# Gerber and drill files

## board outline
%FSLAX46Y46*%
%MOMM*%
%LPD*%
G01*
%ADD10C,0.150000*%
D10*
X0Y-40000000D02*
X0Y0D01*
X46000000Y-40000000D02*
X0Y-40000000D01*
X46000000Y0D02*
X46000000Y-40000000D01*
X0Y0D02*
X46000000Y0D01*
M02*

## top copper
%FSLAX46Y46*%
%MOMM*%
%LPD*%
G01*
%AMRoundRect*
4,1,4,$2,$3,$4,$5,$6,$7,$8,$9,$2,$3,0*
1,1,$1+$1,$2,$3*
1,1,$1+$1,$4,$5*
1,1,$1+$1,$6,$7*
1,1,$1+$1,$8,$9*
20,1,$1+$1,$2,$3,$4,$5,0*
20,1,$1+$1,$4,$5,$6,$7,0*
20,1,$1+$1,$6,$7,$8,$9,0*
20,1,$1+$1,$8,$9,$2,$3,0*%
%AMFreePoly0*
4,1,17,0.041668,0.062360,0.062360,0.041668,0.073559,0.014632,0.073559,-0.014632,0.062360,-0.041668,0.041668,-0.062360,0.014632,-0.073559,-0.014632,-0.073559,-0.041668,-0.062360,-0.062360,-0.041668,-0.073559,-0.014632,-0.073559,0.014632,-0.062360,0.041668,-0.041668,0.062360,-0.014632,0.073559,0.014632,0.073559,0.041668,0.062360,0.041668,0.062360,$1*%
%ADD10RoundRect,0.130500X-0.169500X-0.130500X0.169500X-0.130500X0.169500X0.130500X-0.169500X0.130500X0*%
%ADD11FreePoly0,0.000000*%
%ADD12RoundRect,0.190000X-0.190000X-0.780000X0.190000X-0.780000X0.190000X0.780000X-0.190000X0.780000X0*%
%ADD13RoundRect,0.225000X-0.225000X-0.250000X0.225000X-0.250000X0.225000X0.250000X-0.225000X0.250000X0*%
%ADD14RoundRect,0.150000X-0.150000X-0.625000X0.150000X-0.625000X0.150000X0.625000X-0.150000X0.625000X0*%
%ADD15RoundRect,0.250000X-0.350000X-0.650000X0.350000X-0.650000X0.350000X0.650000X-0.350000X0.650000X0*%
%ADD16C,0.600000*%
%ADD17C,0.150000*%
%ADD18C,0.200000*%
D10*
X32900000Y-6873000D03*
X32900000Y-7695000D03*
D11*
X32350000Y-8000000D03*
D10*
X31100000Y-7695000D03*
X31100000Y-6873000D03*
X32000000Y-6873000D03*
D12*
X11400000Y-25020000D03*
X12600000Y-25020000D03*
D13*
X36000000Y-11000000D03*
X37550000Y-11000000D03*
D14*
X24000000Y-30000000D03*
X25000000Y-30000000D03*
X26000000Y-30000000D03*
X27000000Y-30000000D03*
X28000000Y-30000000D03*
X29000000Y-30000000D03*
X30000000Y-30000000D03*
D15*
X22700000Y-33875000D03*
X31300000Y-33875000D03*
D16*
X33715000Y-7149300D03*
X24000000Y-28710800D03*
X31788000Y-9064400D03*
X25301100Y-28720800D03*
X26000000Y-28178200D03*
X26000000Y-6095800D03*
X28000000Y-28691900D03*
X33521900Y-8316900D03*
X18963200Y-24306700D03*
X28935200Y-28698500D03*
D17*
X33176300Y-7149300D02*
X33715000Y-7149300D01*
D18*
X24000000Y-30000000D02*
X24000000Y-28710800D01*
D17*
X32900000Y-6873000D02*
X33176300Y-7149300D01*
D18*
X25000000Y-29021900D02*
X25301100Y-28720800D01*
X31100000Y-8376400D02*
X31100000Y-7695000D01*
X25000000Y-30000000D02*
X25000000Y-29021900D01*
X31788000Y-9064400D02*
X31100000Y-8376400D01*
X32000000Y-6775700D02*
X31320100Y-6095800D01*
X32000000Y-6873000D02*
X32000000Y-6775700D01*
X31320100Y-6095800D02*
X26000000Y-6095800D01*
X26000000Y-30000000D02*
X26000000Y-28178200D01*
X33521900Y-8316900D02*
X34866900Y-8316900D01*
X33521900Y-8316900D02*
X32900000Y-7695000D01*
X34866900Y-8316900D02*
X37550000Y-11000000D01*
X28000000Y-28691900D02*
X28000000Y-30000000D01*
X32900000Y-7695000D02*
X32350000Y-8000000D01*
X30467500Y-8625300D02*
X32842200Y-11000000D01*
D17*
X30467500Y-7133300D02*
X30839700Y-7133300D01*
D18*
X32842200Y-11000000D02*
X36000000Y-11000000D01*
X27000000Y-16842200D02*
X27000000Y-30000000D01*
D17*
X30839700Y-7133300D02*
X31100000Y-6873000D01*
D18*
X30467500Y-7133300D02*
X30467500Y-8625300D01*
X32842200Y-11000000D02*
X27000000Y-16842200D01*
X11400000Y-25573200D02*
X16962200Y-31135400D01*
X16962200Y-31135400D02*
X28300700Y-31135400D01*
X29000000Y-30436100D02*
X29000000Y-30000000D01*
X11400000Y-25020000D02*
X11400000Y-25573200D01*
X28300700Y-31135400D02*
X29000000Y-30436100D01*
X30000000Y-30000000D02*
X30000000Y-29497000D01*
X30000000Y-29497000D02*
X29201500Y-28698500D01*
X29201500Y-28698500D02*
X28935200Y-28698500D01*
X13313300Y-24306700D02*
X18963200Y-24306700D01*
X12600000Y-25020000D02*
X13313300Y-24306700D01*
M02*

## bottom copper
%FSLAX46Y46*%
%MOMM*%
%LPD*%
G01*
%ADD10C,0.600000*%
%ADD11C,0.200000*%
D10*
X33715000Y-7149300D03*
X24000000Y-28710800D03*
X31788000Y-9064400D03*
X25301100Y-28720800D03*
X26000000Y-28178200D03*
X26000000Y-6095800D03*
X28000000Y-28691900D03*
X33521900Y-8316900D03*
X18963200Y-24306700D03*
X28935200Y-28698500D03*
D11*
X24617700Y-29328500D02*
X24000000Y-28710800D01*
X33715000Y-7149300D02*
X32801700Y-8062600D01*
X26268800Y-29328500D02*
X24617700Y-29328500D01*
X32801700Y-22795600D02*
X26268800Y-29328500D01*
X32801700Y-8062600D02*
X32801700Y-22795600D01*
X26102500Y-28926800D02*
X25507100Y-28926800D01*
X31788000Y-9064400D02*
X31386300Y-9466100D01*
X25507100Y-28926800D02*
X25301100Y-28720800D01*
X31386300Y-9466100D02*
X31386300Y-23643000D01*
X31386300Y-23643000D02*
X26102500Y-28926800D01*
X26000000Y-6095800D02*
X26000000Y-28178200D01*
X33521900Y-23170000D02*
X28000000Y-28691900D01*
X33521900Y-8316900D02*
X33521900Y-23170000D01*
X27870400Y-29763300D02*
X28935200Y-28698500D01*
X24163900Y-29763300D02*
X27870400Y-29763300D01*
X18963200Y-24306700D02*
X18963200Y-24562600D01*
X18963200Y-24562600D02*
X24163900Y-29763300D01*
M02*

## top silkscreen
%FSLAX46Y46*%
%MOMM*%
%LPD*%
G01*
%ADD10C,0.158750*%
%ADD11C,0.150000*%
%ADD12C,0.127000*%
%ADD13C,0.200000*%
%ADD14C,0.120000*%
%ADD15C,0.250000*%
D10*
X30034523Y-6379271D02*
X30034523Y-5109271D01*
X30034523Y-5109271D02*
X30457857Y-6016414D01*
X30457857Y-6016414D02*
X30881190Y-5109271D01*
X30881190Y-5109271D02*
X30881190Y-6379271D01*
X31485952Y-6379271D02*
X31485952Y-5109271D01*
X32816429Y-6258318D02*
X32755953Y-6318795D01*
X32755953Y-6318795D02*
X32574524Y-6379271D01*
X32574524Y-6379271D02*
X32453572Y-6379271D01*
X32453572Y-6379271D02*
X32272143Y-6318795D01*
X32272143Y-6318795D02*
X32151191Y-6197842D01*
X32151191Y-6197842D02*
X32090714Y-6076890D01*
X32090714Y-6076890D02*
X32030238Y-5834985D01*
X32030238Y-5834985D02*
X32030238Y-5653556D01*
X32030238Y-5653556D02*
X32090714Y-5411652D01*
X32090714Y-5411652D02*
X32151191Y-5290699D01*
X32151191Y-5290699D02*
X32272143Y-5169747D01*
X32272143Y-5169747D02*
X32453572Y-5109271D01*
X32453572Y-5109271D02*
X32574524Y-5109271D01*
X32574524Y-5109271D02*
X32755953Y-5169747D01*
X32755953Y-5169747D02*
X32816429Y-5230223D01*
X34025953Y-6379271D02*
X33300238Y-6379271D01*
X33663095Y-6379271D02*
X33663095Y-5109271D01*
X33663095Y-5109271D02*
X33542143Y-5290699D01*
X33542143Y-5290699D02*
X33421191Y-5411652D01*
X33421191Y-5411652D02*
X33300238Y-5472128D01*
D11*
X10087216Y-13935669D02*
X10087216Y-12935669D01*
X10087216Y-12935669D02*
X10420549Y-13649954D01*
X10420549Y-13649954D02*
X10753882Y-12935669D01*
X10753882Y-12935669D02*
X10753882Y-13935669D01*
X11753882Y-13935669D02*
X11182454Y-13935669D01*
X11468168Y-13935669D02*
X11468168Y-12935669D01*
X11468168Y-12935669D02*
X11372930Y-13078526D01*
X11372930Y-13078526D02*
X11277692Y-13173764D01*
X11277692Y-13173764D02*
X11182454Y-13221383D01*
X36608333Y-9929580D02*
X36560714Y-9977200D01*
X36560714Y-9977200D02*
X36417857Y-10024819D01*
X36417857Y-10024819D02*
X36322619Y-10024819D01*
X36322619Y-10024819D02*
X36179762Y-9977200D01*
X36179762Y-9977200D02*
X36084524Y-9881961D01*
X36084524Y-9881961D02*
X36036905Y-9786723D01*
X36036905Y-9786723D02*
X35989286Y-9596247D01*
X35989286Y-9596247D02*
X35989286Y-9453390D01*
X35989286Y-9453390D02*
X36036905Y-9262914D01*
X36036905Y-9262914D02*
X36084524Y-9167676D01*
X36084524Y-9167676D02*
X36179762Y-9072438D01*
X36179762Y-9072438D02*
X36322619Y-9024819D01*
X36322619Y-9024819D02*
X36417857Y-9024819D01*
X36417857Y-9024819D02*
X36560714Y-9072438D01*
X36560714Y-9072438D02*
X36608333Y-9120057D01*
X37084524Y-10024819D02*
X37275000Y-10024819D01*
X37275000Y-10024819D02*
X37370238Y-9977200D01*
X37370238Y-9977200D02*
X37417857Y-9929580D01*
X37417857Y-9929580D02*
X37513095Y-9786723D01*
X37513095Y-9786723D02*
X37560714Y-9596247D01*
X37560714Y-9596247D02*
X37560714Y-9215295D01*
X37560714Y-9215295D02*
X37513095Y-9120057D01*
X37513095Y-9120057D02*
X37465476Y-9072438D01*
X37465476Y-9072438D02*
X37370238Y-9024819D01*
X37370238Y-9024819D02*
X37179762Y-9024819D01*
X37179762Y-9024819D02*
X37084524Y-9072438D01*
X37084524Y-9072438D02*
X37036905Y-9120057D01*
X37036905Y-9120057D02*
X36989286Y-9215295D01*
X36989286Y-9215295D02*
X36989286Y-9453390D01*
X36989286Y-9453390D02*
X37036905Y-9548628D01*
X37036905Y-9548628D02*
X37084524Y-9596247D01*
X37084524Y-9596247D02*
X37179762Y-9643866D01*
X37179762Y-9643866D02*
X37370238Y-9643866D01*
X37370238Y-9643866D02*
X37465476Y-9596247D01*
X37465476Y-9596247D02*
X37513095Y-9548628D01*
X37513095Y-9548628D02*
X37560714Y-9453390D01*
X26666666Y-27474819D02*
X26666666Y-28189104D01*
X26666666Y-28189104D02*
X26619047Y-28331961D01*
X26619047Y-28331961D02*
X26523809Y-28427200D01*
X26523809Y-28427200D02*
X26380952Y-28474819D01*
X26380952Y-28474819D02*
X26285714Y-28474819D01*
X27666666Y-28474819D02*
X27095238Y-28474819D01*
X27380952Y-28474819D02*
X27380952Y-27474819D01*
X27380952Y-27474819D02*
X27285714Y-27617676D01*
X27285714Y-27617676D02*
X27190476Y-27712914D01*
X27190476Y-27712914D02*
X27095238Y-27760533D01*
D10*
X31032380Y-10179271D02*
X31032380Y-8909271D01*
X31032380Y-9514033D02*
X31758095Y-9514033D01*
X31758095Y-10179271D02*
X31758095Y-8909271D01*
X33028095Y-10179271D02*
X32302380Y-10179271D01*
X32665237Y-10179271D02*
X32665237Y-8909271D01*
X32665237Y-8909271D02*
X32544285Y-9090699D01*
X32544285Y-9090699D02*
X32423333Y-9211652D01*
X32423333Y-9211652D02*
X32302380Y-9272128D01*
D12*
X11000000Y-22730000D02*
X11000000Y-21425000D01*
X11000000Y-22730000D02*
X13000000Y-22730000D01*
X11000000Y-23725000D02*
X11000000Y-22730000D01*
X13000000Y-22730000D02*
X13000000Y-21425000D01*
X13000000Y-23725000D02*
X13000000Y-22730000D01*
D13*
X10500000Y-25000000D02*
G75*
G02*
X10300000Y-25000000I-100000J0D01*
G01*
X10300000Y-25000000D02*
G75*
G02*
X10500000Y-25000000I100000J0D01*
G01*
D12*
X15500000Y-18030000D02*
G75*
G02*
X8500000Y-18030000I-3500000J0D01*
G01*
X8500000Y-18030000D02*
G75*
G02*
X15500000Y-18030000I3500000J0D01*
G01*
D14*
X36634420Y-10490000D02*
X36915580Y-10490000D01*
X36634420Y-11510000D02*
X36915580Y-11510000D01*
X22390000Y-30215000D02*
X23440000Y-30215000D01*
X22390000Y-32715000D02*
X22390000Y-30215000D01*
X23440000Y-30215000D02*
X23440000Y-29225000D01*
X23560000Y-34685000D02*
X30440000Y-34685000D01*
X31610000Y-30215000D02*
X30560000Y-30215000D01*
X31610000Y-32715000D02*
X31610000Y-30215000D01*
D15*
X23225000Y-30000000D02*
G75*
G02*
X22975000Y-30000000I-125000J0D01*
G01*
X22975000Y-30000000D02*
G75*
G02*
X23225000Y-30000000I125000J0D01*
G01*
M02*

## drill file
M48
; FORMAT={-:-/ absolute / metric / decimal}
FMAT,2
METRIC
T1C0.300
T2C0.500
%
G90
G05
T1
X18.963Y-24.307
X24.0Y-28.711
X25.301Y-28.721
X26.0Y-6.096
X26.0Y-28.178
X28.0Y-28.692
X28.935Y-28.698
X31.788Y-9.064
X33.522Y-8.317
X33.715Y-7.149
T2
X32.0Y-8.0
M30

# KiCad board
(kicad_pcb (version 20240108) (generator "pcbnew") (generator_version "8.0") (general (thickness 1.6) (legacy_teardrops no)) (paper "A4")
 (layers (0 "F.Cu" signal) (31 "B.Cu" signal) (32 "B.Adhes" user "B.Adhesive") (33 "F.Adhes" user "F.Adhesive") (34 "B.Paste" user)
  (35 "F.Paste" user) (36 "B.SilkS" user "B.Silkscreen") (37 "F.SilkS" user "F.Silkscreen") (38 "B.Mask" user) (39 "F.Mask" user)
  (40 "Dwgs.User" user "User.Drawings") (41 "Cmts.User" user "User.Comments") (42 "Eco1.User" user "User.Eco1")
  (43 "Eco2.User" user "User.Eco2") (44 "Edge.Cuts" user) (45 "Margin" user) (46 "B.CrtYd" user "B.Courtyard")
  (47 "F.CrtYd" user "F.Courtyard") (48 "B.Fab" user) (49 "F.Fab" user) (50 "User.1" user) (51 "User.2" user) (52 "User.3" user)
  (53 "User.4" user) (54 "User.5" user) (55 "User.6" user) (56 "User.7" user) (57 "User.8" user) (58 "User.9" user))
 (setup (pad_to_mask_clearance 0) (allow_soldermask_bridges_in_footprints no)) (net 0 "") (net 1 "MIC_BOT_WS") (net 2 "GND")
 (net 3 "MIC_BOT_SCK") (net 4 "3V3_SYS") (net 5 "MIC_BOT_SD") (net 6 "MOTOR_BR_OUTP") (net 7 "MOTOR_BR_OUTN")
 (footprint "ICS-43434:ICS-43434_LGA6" (layer "F.Cu") (at 32 8)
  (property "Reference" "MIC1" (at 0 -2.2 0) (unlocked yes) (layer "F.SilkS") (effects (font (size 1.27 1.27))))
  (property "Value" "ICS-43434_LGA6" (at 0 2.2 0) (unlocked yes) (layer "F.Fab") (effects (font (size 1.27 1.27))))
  (pad "1" smd roundrect (at 0.9 -1.127) (size 0.6 0.522) (layers "F.Cu" "F.Paste" "F.Mask") (roundrect_rratio 0.25) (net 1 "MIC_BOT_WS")
   (thermal_bridge_angle 45))
  (pad "2" smd roundrect (at 0.9 -0.305) (size 0.6 0.522) (layers "F.Cu" "F.Paste" "F.Mask") (roundrect_rratio 0.25) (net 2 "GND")
   (thermal_bridge_angle 45))
  (pad "3" smd custom (at 0.35 0) (size 0.15 0.15) (layers "F.Cu" "F.Mask") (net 2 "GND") (options (clearance outline) (anchor circle))
   (primitives))
  (pad "4" smd roundrect (at -0.9 -0.305) (size 0.6 0.522) (layers "F.Cu" "F.Paste" "F.Mask") (roundrect_rratio 0.25) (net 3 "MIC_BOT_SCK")
   (thermal_bridge_angle 45))
  (pad "5" smd roundrect (at -0.9 -1.127) (size 0.6 0.522) (layers "F.Cu" "F.Paste" "F.Mask") (roundrect_rratio 0.25) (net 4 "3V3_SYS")
   (thermal_bridge_angle 45))
  (pad "6" smd roundrect (at 0 -1.127) (size 0.6 0.522) (layers "F.Cu" "F.Paste" "F.Mask") (roundrect_rratio 0.25) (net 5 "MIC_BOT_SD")
   (thermal_bridge_angle 45)))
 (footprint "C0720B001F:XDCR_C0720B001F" (layer "F.Cu") (at 12 20)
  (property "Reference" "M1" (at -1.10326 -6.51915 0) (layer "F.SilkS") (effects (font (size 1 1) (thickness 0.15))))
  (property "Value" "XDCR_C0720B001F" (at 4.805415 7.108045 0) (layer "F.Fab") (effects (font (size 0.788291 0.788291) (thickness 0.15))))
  (fp_line (start -1 2.73) (end -1 1.425) (stroke (width 0.127) (type solid)) (layer "F.SilkS"))
  (fp_line (start -1 2.73) (end 1 2.73) (stroke (width 0.127) (type solid)) (layer "F.SilkS"))
  (fp_line (start -1 3.725) (end -1 2.73) (stroke (width 0.127) (type solid)) (layer "F.SilkS"))
  (fp_line (start 1 2.73) (end 1 1.425) (stroke (width 0.127) (type solid)) (layer "F.SilkS"))
  (fp_line (start 1 3.725) (end 1 2.73) (stroke (width 0.127) (type solid)) (layer "F.SilkS"))
  (fp_circle (center -1.6 5) (end -1.5 5) (stroke (width 0.2) (type solid)) (fill none) (layer "F.SilkS"))
  (fp_circle (center 0 -1.97) (end 3.5 -1.97) (stroke (width 0.127) (type solid)) (fill none) (layer "F.SilkS"))
  (pad "1" smd roundrect (at -0.6 5.02) (size 0.76 1.94) (layers "F.Cu" "F.Paste" "F.Mask") (roundrect_rratio 0.25) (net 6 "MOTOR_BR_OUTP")
   (solder_mask_margin 0.102))
  (pad "2" smd roundrect (at 0.6 5.02) (size 0.76 1.94) (layers "F.Cu" "F.Paste" "F.Mask") (roundrect_rratio 0.25) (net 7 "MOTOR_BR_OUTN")
   (solder_mask_margin 0.102)))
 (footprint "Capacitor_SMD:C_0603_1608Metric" (layer "F.Cu") (at 36.775 11)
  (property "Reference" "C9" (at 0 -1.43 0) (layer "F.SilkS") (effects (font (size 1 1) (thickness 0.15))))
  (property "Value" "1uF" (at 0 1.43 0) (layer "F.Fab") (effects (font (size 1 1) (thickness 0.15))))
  (fp_line (start -0.14058 -0.51) (end 0.14058 -0.51) (stroke (width 0.12) (type solid)) (layer "F.SilkS"))
  (fp_line (start -0.14058 0.51) (end 0.14058 0.51) (stroke (width 0.12) (type solid)) (layer "F.SilkS"))
  (pad "1" smd roundrect (at -0.775 0) (size 0.9 0.95) (layers "F.Cu" "F.Paste" "F.Mask") (roundrect_rratio 0.25) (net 4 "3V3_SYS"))
  (pad "2" smd roundrect (at 0.775 0) (size 0.9 0.95) (layers "F.Cu" "F.Paste" "F.Mask") (roundrect_rratio 0.25) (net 2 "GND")))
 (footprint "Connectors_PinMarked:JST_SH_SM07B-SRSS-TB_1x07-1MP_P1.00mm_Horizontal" (layer "F.Cu") (at 27 32)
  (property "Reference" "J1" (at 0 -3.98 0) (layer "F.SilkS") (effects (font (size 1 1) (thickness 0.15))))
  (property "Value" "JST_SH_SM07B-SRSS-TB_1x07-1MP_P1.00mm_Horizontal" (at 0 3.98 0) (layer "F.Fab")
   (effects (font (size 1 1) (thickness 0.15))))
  (fp_line (start -4.61 -1.785) (end -3.56 -1.785) (stroke (width 0.12) (type solid)) (layer "F.SilkS"))
  (fp_line (start -4.61 0.715) (end -4.61 -1.785) (stroke (width 0.12) (type solid)) (layer "F.SilkS"))
  (fp_line (start -3.56 -1.785) (end -3.56 -2.775) (stroke (width 0.12) (type solid)) (layer "F.SilkS"))
  (fp_line (start -3.44 2.685) (end 3.44 2.685) (stroke (width 0.12) (type solid)) (layer "F.SilkS"))
  (fp_line (start 4.61 -1.785) (end 3.56 -1.785) (stroke (width 0.12) (type solid)) (layer "F.SilkS"))
  (fp_line (start 4.61 0.715) (end 4.61 -1.785) (stroke (width 0.12) (type solid)) (layer "F.SilkS"))
  (fp_circle (center -3.9 -2) (end -3.7 -2) (stroke (width 0.1) (type solid)) (fill solid) (layer "F.SilkS"))
  (pad "1" smd roundrect (at -3 -2) (size 0.6 1.55) (layers "F.Cu" "F.Paste" "F.Mask") (roundrect_rratio 0.25) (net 1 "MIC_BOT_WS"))
  (pad "2" smd roundrect (at -2 -2) (size 0.6 1.55) (layers "F.Cu" "F.Paste" "F.Mask") (roundrect_rratio 0.25) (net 3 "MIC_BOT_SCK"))
  (pad "3" smd roundrect (at -1 -2) (size 0.6 1.55) (layers "F.Cu" "F.Paste" "F.Mask") (roundrect_rratio 0.25) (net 5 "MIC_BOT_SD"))
  (pad "4" smd roundrect (at 0 -2) (size 0.6 1.55) (layers "F.Cu" "F.Paste" "F.Mask") (roundrect_rratio 0.25) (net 4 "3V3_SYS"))
  (pad "5" smd roundrect (at 1 -2) (size 0.6 1.55) (layers "F.Cu" "F.Paste" "F.Mask") (roundrect_rratio 0.25) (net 2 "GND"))
  (pad "6" smd roundrect (at 2 -2) (size 0.6 1.55) (layers "F.Cu" "F.Paste" "F.Mask") (roundrect_rratio 0.25) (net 6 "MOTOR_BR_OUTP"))
  (pad "7" smd roundrect (at 3 -2) (size 0.6 1.55) (layers "F.Cu" "F.Paste" "F.Mask") (roundrect_rratio 0.25) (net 7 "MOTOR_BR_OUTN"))
  (pad "MP" smd roundrect (at -4.3 1.875) (size 1.2 1.8) (layers "F.Cu" "F.Paste" "F.Mask") (roundrect_rratio 0.208333))
  (pad "MP" smd roundrect (at 4.3 1.875) (size 1.2 1.8) (layers "F.Cu" "F.Paste" "F.Mask") (roundrect_rratio 0.208333)))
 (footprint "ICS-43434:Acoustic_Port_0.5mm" (layer "F.Cu") (at 32 8)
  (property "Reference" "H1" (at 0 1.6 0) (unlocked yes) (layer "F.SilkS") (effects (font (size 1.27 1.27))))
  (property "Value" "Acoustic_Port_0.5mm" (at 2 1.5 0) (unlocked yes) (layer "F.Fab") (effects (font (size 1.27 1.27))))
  (pad "" np_thru_hole circle (at 0 0) (size 0.5 0.5) (drill 0.5) (layers "*.Cu" "*.Mask")))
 (gr_line (start 0 40) (end 0 0) (stroke (width 0.15) (type default)) (layer "Edge.Cuts"))
 (gr_line (start 46 40) (end 0 40) (stroke (width 0.15) (type default)) (layer "Edge.Cuts"))
 (gr_line (start 46 0) (end 46 40) (stroke (width 0.15) (type default)) (layer "Edge.Cuts"))
 (gr_line (start 0 0) (end 46 0) (stroke (width 0.15) (type default)) (layer "Edge.Cuts"))
 (segment (start 33.1763 7.1493) (end 33.715 7.1493) (width 0.15) (layer "F.Cu") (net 1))
 (segment (start 24 30) (end 24 28.7108) (width 0.2) (layer "F.Cu") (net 1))
 (segment (start 32.9 6.873) (end 33.1763 7.1493) (width 0.15) (layer "F.Cu") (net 1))
 (via (at 33.715 7.1493) (size 0.6) (drill 0.3) (layers "F.Cu" "B.Cu") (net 1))
 (via (at 24 28.7108) (size 0.6) (drill 0.3) (layers "F.Cu" "B.Cu") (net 1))
 (segment (start 24.6177 29.3285) (end 24 28.7108) (width 0.2) (layer "B.Cu") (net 1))
 (segment (start 33.715 7.1493) (end 32.8017 8.0626) (width 0.2) (layer "B.Cu") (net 1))
 (segment (start 26.2688 29.3285) (end 24.6177 29.3285) (width 0.2) (layer "B.Cu") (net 1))
 (segment (start 32.8017 22.7956) (end 26.2688 29.3285) (width 0.2) (layer "B.Cu") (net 1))
 (segment (start 32.8017 8.0626) (end 32.8017 22.7956) (width 0.2) (layer "B.Cu") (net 1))
 (segment (start 25 29.0219) (end 25.3011 28.7208) (width 0.2) (layer "F.Cu") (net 3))
 (segment (start 31.1 8.3764) (end 31.1 7.695) (width 0.2) (layer "F.Cu") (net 3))
 (segment (start 25 30) (end 25 29.0219) (width 0.2) (layer "F.Cu") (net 3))
 (segment (start 31.788 9.0644) (end 31.1 8.3764) (width 0.2) (layer "F.Cu") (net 3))
 (via (at 31.788 9.0644) (size 0.6) (drill 0.3) (layers "F.Cu" "B.Cu") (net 3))
 (via (at 25.3011 28.7208) (size 0.6) (drill 0.3) (layers "F.Cu" "B.Cu") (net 3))
 (segment (start 26.1025 28.9268) (end 25.5071 28.9268) (width 0.2) (layer "B.Cu") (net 3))
 (segment (start 31.788 9.0644) (end 31.3863 9.4661) (width 0.2) (layer "B.Cu") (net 3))
 (segment (start 25.5071 28.9268) (end 25.3011 28.7208) (width 0.2) (layer "B.Cu") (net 3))
 (segment (start 31.3863 9.4661) (end 31.3863 23.643) (width 0.2) (layer "B.Cu") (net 3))
 (segment (start 31.3863 23.643) (end 26.1025 28.9268) (width 0.2) (layer "B.Cu") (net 3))
 (segment (start 32 6.7757) (end 31.3201 6.0958) (width 0.2) (layer "F.Cu") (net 5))
 (segment (start 32 6.873) (end 32 6.7757) (width 0.2) (layer "F.Cu") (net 5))
 (segment (start 31.3201 6.0958) (end 26 6.0958) (width 0.2) (layer "F.Cu") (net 5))
 (segment (start 26 30) (end 26 28.1782) (width 0.2) (layer "F.Cu") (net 5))
 (via (at 26 28.1782) (size 0.6) (drill 0.3) (layers "F.Cu" "B.Cu") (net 5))
 (via (at 26 6.0958) (size 0.6) (drill 0.3) (layers "F.Cu" "B.Cu") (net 5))
 (segment (start 26 6.0958) (end 26 28.1782) (width 0.2) (layer "B.Cu") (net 5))
 (segment (start 33.5219 8.3169) (end 34.8669 8.3169) (width 0.2) (layer "F.Cu") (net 2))
 (segment (start 33.5219 8.3169) (end 32.9 7.695) (width 0.2) (layer "F.Cu") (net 2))
 (segment (start 34.8669 8.3169) (end 37.55 11) (width 0.2) (layer "F.Cu") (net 2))
 (segment (start 28 28.6919) (end 28 30) (width 0.2) (layer "F.Cu") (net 2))
 (segment (start 32.9 7.695) (end 32.35 8) (width 0.2) (layer "F.Cu") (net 2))
 (via (at 28 28.6919) (size 0.6) (drill 0.3) (layers "F.Cu" "B.Cu") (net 2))
 (via (at 33.5219 8.3169) (size 0.6) (drill 0.3) (layers "F.Cu" "B.Cu") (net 2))
 (segment (start 33.5219 23.17) (end 28 28.6919) (width 0.2) (layer "B.Cu") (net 2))
 (segment (start 33.5219 8.3169) (end 33.5219 23.17) (width 0.2) (layer "B.Cu") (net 2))
 (segment (start 30.4675 8.6253) (end 32.8422 11) (width 0.2) (layer "F.Cu") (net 4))
 (segment (start 30.4675 7.1333) (end 30.8397 7.1333) (width 0.15) (layer "F.Cu") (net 4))
 (segment (start 32.8422 11) (end 36 11) (width 0.2) (layer "F.Cu") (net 4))
 (segment (start 27 16.8422) (end 27 30) (width 0.2) (layer "F.Cu") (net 4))
 (segment (start 30.8397 7.1333) (end 31.1 6.873) (width 0.15) (layer "F.Cu") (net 4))
 (segment (start 30.4675 7.1333) (end 30.4675 8.6253) (width 0.2) (layer "F.Cu") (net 4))
 (segment (start 32.8422 11) (end 27 16.8422) (width 0.2) (layer "F.Cu") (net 4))
 (segment (start 11.4 25.5732) (end 16.9622 31.1354) (width 0.2) (layer "F.Cu") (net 6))
 (segment (start 16.9622 31.1354) (end 28.3007 31.1354) (width 0.2) (layer "F.Cu") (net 6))
 (segment (start 29 30.4361) (end 29 30) (width 0.2) (layer "F.Cu") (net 6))
 (segment (start 11.4 25.02) (end 11.4 25.5732) (width 0.2) (layer "F.Cu") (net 6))
 (segment (start 28.3007 31.1354) (end 29 30.4361) (width 0.2) (layer "F.Cu") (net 6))
 (segment (start 30 30) (end 30 29.497) (width 0.2) (layer "F.Cu") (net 7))
 (segment (start 30 29.497) (end 29.2015 28.6985) (width 0.2) (layer "F.Cu") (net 7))
 (segment (start 29.2015 28.6985) (end 28.9352 28.6985) (width 0.2) (layer "F.Cu") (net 7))
 (segment (start 13.3133 24.3067) (end 18.9632 24.3067) (width 0.2) (layer "F.Cu") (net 7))
 (segment (start 12.6 25.02) (end 13.3133 24.3067) (width 0.2) (layer "F.Cu") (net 7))
 (via (at 18.9632 24.3067) (size 0.6) (drill 0.3) (layers "F.Cu" "B.Cu") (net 7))
 (via (at 28.9352 28.6985) (size 0.6) (drill 0.3) (layers "F.Cu" "B.Cu") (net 7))
 (segment (start 27.8704 29.7633) (end 28.9352 28.6985) (width 0.2) (layer "B.Cu") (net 7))
 (segment (start 24.1639 29.7633) (end 27.8704 29.7633) (width 0.2) (layer "B.Cu") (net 7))
 (segment (start 18.9632 24.3067) (end 18.9632 24.5626) (width 0.2) (layer "B.Cu") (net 7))
 (segment (start 18.9632 24.5626) (end 24.1639 29.7633) (width 0.2) (layer "B.Cu") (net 7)))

